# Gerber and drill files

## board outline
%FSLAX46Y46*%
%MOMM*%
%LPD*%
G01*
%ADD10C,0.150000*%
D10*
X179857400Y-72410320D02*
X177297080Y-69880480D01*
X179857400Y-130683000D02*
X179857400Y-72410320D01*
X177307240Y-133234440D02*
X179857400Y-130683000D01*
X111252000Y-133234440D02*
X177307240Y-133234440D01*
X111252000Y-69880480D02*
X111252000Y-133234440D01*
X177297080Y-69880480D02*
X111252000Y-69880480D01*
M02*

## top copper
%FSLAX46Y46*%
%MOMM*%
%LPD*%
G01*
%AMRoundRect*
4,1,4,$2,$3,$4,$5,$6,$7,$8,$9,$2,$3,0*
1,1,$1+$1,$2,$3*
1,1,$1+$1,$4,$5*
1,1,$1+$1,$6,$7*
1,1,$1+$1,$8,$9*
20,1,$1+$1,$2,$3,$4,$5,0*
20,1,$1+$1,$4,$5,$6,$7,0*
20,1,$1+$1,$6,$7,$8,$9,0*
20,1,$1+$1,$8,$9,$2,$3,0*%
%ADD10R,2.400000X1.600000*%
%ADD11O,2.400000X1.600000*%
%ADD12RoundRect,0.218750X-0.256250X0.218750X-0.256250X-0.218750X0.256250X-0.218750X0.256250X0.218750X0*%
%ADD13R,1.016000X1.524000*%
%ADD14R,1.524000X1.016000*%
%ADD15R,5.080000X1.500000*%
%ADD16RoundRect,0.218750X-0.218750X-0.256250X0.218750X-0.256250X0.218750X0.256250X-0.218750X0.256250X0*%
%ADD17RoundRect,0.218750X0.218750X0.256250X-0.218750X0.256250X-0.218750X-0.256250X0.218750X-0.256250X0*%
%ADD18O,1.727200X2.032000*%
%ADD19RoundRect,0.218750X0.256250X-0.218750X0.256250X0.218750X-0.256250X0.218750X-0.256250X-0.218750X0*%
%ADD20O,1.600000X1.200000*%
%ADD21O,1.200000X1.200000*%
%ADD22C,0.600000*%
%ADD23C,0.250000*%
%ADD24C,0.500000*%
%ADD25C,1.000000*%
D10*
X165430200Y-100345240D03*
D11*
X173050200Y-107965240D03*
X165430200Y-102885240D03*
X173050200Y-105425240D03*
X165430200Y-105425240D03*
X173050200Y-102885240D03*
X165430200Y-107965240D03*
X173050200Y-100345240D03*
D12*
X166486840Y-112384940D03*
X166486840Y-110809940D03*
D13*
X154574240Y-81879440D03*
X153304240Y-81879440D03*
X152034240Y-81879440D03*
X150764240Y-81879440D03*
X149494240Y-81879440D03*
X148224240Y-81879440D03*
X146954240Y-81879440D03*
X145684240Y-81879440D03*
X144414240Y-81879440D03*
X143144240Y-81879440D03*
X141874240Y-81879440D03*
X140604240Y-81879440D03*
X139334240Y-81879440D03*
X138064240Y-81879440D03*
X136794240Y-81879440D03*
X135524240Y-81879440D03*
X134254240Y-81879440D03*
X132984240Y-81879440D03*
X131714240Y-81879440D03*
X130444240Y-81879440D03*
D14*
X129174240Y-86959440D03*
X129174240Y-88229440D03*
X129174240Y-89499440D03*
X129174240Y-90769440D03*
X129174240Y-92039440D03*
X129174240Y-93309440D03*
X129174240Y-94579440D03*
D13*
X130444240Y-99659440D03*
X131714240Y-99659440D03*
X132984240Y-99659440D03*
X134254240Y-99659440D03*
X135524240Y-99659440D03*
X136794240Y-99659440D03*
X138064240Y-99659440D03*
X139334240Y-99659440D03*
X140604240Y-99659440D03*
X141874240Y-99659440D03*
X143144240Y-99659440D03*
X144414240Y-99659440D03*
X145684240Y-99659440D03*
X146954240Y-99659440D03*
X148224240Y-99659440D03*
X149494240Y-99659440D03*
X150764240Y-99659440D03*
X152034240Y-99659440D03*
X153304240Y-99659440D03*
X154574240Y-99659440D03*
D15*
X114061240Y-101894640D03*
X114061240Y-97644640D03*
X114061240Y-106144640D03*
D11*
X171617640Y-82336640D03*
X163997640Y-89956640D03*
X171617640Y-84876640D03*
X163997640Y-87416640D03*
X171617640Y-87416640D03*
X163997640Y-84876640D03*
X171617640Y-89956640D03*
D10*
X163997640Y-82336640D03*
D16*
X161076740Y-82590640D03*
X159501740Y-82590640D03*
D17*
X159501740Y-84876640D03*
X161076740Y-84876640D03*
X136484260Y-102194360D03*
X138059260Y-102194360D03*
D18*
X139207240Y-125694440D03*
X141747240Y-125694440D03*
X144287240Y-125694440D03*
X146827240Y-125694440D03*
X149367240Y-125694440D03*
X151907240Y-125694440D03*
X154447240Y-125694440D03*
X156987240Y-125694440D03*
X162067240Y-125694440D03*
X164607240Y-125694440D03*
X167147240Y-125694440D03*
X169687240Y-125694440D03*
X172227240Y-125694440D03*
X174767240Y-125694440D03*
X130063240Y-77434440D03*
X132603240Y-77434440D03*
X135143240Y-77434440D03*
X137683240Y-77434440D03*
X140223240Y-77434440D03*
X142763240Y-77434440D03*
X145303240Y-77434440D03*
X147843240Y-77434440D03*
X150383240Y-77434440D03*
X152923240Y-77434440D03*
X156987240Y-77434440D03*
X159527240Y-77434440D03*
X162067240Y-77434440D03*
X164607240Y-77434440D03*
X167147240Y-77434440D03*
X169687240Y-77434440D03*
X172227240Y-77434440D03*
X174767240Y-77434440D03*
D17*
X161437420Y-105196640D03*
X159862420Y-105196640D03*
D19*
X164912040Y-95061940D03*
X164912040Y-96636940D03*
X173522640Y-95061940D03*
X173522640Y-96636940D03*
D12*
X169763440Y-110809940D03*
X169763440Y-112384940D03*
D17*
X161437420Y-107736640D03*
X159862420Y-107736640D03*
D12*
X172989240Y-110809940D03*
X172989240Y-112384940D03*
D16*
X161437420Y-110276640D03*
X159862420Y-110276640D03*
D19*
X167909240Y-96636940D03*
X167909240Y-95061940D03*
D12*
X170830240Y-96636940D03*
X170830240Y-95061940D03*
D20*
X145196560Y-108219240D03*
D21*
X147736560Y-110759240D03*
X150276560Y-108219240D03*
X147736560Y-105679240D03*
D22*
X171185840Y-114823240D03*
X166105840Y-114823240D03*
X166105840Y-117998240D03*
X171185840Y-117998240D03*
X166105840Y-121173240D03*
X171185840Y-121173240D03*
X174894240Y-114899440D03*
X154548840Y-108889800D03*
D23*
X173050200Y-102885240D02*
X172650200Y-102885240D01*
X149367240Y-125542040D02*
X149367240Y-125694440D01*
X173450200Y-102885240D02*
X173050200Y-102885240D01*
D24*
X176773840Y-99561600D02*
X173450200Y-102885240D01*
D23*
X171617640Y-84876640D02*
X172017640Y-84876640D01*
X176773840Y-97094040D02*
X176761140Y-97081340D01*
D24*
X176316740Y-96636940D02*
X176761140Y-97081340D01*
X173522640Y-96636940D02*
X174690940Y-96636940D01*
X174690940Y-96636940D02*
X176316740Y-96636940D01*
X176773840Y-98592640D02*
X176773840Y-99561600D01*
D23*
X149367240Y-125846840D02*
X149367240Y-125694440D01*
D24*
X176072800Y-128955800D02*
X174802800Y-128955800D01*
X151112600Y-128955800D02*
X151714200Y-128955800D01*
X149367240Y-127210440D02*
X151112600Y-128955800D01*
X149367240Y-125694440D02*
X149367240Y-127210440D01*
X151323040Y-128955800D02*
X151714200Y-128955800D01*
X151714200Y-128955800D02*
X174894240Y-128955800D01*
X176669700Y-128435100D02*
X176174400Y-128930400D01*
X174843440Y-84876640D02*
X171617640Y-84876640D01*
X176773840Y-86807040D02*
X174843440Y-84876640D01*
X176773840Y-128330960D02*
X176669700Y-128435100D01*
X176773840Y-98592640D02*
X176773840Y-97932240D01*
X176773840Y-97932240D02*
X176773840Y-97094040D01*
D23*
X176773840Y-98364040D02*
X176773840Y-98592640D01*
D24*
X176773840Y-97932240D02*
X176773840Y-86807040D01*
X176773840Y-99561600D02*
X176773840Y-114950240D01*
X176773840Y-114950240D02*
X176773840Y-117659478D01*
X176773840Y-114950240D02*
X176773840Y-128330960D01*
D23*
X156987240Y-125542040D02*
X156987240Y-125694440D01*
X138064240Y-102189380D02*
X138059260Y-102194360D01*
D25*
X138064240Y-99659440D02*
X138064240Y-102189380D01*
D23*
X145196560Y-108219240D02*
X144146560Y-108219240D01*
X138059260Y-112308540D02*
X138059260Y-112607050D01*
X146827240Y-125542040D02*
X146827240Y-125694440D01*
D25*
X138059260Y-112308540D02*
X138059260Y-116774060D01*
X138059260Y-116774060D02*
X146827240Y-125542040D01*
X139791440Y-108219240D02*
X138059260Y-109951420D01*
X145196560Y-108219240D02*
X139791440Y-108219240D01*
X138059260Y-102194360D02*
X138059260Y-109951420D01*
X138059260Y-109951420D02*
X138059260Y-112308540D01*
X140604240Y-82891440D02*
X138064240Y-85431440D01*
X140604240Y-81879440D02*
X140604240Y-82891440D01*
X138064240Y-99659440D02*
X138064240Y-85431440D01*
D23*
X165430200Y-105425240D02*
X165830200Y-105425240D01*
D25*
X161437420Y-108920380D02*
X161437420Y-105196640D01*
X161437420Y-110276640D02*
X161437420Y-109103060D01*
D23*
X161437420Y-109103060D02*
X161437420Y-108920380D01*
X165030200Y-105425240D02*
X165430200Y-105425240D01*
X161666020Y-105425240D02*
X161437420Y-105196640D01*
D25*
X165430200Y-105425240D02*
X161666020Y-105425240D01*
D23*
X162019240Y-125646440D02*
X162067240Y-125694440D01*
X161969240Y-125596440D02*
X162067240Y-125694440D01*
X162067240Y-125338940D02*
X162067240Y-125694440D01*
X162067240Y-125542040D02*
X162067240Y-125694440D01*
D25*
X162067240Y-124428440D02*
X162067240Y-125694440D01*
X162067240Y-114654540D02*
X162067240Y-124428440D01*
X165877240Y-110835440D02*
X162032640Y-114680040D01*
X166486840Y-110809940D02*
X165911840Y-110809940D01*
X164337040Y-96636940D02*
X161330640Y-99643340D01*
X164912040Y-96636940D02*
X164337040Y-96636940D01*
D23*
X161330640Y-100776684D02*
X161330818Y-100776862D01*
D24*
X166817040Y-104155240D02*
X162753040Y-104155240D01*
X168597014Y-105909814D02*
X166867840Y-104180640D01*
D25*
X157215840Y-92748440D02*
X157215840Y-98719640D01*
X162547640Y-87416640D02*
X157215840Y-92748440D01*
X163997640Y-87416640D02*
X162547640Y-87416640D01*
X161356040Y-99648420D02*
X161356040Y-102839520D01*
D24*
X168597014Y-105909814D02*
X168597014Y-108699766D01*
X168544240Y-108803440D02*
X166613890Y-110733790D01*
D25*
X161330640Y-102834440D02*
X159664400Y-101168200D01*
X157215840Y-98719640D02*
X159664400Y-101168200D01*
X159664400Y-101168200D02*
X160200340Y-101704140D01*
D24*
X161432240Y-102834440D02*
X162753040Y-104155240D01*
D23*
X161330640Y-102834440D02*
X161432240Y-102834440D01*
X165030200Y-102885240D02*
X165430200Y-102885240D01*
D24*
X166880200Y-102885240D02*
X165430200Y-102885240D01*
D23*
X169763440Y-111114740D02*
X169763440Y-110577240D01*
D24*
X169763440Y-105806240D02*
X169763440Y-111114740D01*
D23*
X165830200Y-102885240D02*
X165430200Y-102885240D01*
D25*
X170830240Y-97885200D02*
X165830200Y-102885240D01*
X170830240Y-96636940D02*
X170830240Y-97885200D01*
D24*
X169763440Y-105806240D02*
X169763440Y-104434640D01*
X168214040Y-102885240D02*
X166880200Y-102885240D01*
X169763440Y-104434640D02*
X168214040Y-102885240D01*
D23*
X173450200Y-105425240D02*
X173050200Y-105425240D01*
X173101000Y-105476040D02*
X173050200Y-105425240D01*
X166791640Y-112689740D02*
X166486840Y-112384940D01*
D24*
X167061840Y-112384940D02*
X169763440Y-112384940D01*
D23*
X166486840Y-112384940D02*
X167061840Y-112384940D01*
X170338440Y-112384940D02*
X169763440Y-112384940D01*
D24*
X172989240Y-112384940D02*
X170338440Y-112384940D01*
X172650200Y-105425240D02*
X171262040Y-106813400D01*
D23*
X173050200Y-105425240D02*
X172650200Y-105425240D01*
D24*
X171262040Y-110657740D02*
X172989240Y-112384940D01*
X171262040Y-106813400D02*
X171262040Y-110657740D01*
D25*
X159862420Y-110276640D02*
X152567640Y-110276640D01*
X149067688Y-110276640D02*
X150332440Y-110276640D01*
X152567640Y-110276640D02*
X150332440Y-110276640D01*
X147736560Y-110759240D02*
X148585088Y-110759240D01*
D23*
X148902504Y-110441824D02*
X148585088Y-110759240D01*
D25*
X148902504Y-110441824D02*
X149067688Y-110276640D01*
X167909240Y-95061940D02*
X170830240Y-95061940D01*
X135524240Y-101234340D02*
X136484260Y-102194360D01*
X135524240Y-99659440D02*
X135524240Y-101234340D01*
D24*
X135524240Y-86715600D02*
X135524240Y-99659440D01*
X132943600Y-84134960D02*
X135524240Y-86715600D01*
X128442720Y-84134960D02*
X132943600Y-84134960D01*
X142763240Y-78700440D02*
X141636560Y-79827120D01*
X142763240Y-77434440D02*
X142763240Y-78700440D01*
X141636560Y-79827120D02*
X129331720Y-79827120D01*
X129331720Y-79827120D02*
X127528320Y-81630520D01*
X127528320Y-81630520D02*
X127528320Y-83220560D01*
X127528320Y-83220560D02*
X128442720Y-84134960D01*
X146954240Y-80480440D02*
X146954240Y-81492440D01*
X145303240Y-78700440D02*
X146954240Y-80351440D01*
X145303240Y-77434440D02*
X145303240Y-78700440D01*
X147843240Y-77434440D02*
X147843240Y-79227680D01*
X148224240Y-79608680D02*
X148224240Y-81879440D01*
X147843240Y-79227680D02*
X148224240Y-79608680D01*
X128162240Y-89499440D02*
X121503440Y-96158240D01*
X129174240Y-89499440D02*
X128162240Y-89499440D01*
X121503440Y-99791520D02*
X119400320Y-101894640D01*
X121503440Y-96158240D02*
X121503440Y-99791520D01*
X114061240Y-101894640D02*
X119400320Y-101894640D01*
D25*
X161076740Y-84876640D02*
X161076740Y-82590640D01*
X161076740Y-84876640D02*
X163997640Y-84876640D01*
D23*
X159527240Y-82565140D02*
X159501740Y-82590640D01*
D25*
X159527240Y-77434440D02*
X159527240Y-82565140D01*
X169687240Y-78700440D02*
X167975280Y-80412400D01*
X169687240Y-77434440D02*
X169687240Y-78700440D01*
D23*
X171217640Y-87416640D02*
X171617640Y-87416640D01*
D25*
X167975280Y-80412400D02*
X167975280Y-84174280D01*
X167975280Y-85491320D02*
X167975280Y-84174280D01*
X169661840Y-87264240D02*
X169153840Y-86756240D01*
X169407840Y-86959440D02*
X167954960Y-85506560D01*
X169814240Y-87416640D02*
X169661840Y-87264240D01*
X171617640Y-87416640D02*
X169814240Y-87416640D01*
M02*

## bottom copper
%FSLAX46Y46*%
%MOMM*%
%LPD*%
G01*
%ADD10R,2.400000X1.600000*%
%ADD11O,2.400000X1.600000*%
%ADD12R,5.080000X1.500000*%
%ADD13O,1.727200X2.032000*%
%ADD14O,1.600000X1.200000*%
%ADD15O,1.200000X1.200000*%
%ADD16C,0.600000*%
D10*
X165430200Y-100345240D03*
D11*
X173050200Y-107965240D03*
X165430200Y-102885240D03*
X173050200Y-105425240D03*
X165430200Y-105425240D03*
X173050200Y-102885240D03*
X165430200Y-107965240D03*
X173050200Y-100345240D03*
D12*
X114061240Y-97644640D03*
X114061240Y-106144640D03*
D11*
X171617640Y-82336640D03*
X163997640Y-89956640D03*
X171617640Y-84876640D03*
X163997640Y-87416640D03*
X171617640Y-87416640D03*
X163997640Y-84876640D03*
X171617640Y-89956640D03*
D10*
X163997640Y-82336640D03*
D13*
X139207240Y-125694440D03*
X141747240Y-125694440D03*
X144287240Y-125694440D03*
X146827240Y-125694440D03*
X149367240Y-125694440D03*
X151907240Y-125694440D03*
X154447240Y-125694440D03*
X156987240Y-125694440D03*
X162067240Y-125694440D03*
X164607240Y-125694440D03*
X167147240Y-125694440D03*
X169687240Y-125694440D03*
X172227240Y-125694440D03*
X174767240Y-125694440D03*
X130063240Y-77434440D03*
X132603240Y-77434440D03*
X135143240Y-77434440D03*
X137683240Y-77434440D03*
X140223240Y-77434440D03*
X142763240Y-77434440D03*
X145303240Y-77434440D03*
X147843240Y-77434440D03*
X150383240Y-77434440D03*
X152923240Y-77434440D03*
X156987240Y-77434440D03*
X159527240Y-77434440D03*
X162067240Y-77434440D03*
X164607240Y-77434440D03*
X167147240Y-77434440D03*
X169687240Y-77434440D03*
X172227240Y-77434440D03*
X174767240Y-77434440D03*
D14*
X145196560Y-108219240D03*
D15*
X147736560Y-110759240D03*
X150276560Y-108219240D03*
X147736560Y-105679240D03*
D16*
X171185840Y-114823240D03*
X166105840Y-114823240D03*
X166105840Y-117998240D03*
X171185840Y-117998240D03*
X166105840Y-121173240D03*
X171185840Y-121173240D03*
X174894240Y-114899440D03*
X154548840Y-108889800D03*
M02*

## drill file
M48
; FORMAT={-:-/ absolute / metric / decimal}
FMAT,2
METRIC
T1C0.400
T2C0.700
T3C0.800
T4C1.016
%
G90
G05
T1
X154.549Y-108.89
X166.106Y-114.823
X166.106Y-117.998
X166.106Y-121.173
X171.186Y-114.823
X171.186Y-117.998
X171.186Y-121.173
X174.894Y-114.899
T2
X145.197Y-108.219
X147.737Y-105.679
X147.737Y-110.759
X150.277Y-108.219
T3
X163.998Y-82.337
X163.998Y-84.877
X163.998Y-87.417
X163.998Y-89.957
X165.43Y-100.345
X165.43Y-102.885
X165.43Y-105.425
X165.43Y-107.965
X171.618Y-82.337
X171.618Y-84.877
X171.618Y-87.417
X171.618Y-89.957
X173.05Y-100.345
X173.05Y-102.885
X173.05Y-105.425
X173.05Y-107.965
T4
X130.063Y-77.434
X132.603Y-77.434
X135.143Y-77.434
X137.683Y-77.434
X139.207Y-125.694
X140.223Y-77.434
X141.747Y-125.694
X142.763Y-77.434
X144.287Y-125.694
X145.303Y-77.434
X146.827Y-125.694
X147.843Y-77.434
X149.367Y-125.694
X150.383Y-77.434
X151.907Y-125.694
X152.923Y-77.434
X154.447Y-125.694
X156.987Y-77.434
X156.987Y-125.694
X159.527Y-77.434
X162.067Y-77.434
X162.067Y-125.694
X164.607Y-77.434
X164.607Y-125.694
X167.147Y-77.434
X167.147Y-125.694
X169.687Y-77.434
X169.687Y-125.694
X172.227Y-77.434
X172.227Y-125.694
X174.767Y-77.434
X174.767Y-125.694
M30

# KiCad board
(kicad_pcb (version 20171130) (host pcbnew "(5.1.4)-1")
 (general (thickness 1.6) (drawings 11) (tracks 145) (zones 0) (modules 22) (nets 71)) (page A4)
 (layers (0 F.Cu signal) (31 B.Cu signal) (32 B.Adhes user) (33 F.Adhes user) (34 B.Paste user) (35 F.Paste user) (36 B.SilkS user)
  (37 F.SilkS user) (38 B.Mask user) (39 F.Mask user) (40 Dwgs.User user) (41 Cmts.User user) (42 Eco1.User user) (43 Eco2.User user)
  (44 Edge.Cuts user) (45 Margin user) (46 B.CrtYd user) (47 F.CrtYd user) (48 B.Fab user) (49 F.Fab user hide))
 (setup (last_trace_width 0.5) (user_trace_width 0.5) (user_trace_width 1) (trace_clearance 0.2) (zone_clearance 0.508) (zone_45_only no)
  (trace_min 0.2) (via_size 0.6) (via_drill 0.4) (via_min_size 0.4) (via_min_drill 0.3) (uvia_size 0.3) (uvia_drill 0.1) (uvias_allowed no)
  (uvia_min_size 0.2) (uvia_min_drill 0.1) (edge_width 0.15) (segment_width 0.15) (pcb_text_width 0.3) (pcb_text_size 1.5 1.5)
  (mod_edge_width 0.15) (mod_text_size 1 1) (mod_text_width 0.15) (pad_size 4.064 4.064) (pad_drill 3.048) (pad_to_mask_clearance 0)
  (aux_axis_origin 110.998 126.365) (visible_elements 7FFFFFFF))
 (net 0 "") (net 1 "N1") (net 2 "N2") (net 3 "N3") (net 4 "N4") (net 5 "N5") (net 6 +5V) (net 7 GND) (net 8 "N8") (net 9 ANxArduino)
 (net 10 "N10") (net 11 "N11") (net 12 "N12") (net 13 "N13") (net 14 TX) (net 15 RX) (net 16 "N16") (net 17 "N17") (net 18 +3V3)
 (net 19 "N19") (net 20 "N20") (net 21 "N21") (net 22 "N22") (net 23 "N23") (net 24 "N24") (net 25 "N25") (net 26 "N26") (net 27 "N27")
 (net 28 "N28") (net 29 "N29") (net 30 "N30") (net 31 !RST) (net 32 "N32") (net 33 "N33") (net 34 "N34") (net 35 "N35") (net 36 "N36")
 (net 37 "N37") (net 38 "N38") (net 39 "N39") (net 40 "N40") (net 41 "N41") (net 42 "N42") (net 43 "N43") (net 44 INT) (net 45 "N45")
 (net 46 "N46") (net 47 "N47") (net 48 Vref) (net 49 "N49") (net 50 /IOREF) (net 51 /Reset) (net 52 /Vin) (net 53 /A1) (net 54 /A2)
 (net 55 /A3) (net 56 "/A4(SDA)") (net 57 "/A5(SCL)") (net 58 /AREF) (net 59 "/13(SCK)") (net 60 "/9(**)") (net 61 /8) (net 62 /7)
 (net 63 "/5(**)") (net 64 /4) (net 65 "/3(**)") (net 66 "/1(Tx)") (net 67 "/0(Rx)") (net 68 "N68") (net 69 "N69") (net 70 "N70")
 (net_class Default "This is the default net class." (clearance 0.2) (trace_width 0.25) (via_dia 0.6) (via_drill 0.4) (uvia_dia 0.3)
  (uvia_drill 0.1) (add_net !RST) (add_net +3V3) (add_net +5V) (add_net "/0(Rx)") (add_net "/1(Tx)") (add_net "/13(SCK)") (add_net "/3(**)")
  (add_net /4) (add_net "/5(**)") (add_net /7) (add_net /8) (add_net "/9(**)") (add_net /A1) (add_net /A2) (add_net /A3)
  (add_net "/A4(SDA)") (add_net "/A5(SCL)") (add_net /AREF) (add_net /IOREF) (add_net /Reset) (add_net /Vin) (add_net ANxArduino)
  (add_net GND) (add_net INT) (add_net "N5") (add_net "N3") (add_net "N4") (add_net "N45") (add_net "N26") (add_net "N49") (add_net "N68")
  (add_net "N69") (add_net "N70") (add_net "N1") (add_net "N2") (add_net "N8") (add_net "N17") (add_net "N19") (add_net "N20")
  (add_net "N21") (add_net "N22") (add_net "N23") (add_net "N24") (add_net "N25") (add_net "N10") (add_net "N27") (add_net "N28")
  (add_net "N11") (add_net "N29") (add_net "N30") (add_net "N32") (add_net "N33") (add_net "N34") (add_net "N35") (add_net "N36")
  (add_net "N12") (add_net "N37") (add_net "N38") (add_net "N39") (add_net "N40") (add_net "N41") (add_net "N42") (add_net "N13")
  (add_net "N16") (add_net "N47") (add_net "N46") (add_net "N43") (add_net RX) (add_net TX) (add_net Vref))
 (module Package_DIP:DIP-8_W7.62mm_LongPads (layer F.Cu) (at 165.4302 100.34524)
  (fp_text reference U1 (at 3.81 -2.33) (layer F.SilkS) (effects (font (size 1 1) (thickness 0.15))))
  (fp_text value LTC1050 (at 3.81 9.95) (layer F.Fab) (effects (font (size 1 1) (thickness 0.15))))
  (pad 1 thru_hole rect (at 0 0) (size 2.4 1.6) (drill 0.8) (layers *.Cu *.Mask) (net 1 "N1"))
  (pad 5 thru_hole oval (at 7.62 7.62) (size 2.4 1.6) (drill 0.8) (layers *.Cu *.Mask) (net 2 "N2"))
  (pad 2 thru_hole oval (at 0 2.54) (size 2.4 1.6) (drill 0.8) (layers *.Cu *.Mask) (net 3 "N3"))
  (pad 6 thru_hole oval (at 7.62 5.08) (size 2.4 1.6) (drill 0.8) (layers *.Cu *.Mask) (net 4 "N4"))
  (pad 3 thru_hole oval (at 0 5.08) (size 2.4 1.6) (drill 0.8) (layers *.Cu *.Mask) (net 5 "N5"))
  (pad 7 thru_hole oval (at 7.62 2.54) (size 2.4 1.6) (drill 0.8) (layers *.Cu *.Mask) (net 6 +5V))
  (pad 4 thru_hole oval (at 0 7.62) (size 2.4 1.6) (drill 0.8) (layers *.Cu *.Mask) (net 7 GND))
  (pad 8 thru_hole oval (at 7.62 0) (size 2.4 1.6) (drill 0.8) (layers *.Cu *.Mask) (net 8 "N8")))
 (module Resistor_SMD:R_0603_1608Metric (layer F.Cu) (at 166.48684 111.59744 270)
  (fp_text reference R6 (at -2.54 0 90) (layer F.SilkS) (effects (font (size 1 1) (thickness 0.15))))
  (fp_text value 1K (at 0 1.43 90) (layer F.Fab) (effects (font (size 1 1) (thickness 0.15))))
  (pad 2 smd roundrect (at 0.7875 0 270) (size 0.875 0.95) (layers F.Cu F.Paste F.Mask) (roundrect_rratio 0.25) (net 4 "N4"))
  (pad 1 smd roundrect (at -0.7875 0 270) (size 0.875 0.95) (layers F.Cu F.Paste F.Mask) (roundrect_rratio 0.25) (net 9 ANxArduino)))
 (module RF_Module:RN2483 (layer F.Cu) (at 142.50924 90.76944 270)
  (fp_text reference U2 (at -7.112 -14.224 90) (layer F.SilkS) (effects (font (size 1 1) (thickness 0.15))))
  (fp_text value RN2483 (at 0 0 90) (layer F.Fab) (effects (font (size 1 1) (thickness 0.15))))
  (pad 1 smd rect (at -8.89 -12.065 270) (size 1.524 1.016) (layers F.Cu F.Paste F.Mask) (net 7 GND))
  (pad 2 smd rect (at -8.89 -10.795 270) (size 1.524 1.016) (layers F.Cu F.Paste F.Mask) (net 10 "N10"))
  (pad 3 smd rect (at -8.89 -9.525 270) (size 1.524 1.016) (layers F.Cu F.Paste F.Mask) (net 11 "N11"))
  (pad 4 smd rect (at -8.89 -8.255 270) (size 1.524 1.016) (layers F.Cu F.Paste F.Mask) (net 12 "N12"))
  (pad 5 smd rect (at -8.89 -6.985 270) (size 1.524 1.016) (layers F.Cu F.Paste F.Mask) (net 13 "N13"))
  (pad 6 smd rect (at -8.89 -5.715 270) (size 1.524 1.016) (layers F.Cu F.Paste F.Mask) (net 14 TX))
  (pad 7 smd rect (at -8.89 -4.445 270) (size 1.524 1.016) (layers F.Cu F.Paste F.Mask) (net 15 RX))
  (pad 8 smd rect (at -8.89 -3.175 270) (size 1.524 1.016) (layers F.Cu F.Paste F.Mask) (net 7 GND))
  (pad 9 smd rect (at -8.89 -1.905 270) (size 1.524 1.016) (layers F.Cu F.Paste F.Mask) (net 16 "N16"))
  (pad 10 smd rect (at -8.89 -0.635 270) (size 1.524 1.016) (layers F.Cu F.Paste F.Mask) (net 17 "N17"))
  (pad 11 smd rect (at -8.89 0.635 270) (size 1.524 1.016) (layers F.Cu F.Paste F.Mask) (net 7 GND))
  (pad 12 smd rect (at -8.89 1.905 270) (size 1.524 1.016) (layers F.Cu F.Paste F.Mask) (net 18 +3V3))
  (pad 13 smd rect (at -8.89 3.175 270) (size 1.524 1.016) (layers F.Cu F.Paste F.Mask) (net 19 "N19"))
  (pad 14 smd rect (at -8.89 4.445 270) (size 1.524 1.016) (layers F.Cu F.Paste F.Mask) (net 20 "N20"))
  (pad 15 smd rect (at -8.89 5.715 270) (size 1.524 1.016) (layers F.Cu F.Paste F.Mask) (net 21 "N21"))
  (pad 16 smd rect (at -8.89 6.985 270) (size 1.524 1.016) (layers F.Cu F.Paste F.Mask) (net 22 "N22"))
  (pad 17 smd rect (at -8.89 8.255 270) (size 1.524 1.016) (layers F.Cu F.Paste F.Mask) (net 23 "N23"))
  (pad 18 smd rect (at -8.89 9.525 270) (size 1.524 1.016) (layers F.Cu F.Paste F.Mask) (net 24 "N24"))
  (pad 19 smd rect (at -8.89 10.795 270) (size 1.524 1.016) (layers F.Cu F.Paste F.Mask) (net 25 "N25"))
  (pad 20 smd rect (at -8.89 12.065 270) (size 1.524 1.016) (layers F.Cu F.Paste F.Mask) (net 7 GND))
  (pad 21 smd rect (at -3.81 13.335) (size 1.524 1.016) (layers F.Cu F.Paste F.Mask) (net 7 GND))
  (pad 22 smd rect (at -2.54 13.335) (size 1.524 1.016) (layers F.Cu F.Paste F.Mask) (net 7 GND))
  (pad 23 smd rect (at -1.27 13.335) (size 1.524 1.016) (layers F.Cu F.Paste F.Mask) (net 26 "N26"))
  (pad 24 smd rect (at 0 13.335) (size 1.524 1.016) (layers F.Cu F.Paste F.Mask) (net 7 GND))
  (pad 25 smd rect (at 1.27 13.335) (size 1.524 1.016) (layers F.Cu F.Paste F.Mask) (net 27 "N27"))
  (pad 26 smd rect (at 2.54 13.335) (size 1.524 1.016) (layers F.Cu F.Paste F.Mask) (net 7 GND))
  (pad 27 smd rect (at 3.81 13.335) (size 1.524 1.016) (layers F.Cu F.Paste F.Mask) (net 7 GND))
  (pad 28 smd rect (at 8.89 12.065 270) (size 1.524 1.016) (layers F.Cu F.Paste F.Mask) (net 7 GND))
  (pad 29 smd rect (at 8.89 10.795 270) (size 1.524 1.016) (layers F.Cu F.Paste F.Mask) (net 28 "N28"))
  (pad 30 smd rect (at 8.89 9.525 270) (size 1.524 1.016) (layers F.Cu F.Paste F.Mask) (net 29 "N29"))
  (pad 31 smd rect (at 8.89 8.255 270) (size 1.524 1.016) (layers F.Cu F.Paste F.Mask) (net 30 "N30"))
  (pad 32 smd rect (at 8.89 6.985 270) (size 1.524 1.016) (layers F.Cu F.Paste F.Mask) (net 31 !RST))
  (pad 33 smd rect (at 8.89 5.715 270) (size 1.524 1.016) (layers F.Cu F.Paste F.Mask) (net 7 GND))
  (pad 34 smd rect (at 8.89 4.445 270) (size 1.524 1.016) (layers F.Cu F.Paste F.Mask) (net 18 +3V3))
  (pad 35 smd rect (at 8.89 3.175 270) (size 1.524 1.016) (layers F.Cu F.Paste F.Mask) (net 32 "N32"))
  (pad 36 smd rect (at 8.89 1.905 270) (size 1.524 1.016) (layers F.Cu F.Paste F.Mask) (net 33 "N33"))
  (pad 37 smd rect (at 8.89 0.635 270) (size 1.524 1.016) (layers F.Cu F.Paste F.Mask) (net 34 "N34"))
  (pad 38 smd rect (at 8.89 -0.635 270) (size 1.524 1.016) (layers F.Cu F.Paste F.Mask) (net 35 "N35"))
  (pad 39 smd rect (at 8.89 -1.905 270) (size 1.524 1.016) (layers F.Cu F.Paste F.Mask) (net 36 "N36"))
  (pad 40 smd rect (at 8.89 -3.175 270) (size 1.524 1.016) (layers F.Cu F.Paste F.Mask) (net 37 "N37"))
  (pad 41 smd rect (at 8.89 -4.445 270) (size 1.524 1.016) (layers F.Cu F.Paste F.Mask) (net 7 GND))
  (pad 42 smd rect (at 8.89 -5.715 270) (size 1.524 1.016) (layers F.Cu F.Paste F.Mask) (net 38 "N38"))
  (pad 43 smd rect (at 8.89 -6.985 270) (size 1.524 1.016) (layers F.Cu F.Paste F.Mask) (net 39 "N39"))
  (pad 44 smd rect (at 8.89 -8.255 270) (size 1.524 1.016) (layers F.Cu F.Paste F.Mask) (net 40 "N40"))
  (pad 45 smd rect (at 8.89 -9.525 270) (size 1.524 1.016) (layers F.Cu F.Paste F.Mask) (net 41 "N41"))
  (pad 46 smd rect (at 8.89 -10.795 270) (size 1.524 1.016) (layers F.Cu F.Paste F.Mask) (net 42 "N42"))
  (pad 47 smd rect (at 8.89 -12.065 270) (size 1.524 1.016) (layers F.Cu F.Paste F.Mask) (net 7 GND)))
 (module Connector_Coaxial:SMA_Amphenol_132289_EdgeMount (layer F.Cu) (at 114.06124 101.89464)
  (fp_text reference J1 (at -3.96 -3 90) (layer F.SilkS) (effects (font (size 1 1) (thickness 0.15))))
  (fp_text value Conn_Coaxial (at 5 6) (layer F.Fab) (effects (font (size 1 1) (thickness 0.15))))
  (pad 1 smd rect (at 0 0 90) (size 1.5 5.08) (layers F.Cu F.Paste F.Mask) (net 26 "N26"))
  (pad 2 smd rect (at 0 -4.25 90) (size 1.5 5.08) (layers F.Cu F.Paste F.Mask) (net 7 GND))
  (pad 2 smd rect (at 0 4.25 90) (size 1.5 5.08) (layers F.Cu F.Paste F.Mask) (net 7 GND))
  (pad 2 smd rect (at 0 -4.25 90) (size 1.5 5.08) (layers B.Cu B.Paste B.Mask) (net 7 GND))
  (pad 2 smd rect (at 0 4.25 90) (size 1.5 5.08) (layers B.Cu B.Paste B.Mask) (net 7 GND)))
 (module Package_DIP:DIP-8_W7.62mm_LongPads (layer F.Cu) (at 163.99764 82.33664)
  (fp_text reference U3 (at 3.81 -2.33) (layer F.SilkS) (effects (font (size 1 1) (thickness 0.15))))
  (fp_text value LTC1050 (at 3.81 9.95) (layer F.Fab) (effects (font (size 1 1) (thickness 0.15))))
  (pad 8 thru_hole oval (at 7.62 0) (size 2.4 1.6) (drill 0.8) (layers *.Cu *.Mask) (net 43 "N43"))
  (pad 4 thru_hole oval (at 0 7.62) (size 2.4 1.6) (drill 0.8) (layers *.Cu *.Mask) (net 7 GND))
  (pad 7 thru_hole oval (at 7.62 2.54) (size 2.4 1.6) (drill 0.8) (layers *.Cu *.Mask) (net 6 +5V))
  (pad 3 thru_hole oval (at 0 5.08) (size 2.4 1.6) (drill 0.8) (layers *.Cu *.Mask) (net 9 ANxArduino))
  (pad 6 thru_hole oval (at 7.62 5.08) (size 2.4 1.6) (drill 0.8) (layers *.Cu *.Mask) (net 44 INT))
  (pad 2 thru_hole oval (at 0 2.54) (size 2.4 1.6) (drill 0.8) (layers *.Cu *.Mask) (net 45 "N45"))
  (pad 5 thru_hole oval (at 7.62 7.62) (size 2.4 1.6) (drill 0.8) (layers *.Cu *.Mask) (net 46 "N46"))
  (pad 1 thru_hole rect (at 0 0) (size 2.4 1.6) (drill 0.8) (layers *.Cu *.Mask) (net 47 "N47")))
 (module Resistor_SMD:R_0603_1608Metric (layer F.Cu) (at 160.28924 82.59064)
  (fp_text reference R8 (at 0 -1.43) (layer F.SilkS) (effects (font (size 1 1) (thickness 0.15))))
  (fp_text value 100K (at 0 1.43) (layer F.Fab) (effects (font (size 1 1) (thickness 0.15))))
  (pad 2 smd roundrect (at 0.7875 0) (size 0.875 0.95) (layers F.Cu F.Paste F.Mask) (roundrect_rratio 0.25) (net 45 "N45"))
  (pad 1 smd roundrect (at -0.7875 0) (size 0.875 0.95) (layers F.Cu F.Paste F.Mask) (roundrect_rratio 0.25) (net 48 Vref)))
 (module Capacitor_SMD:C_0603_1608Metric (layer F.Cu) (at 160.28924 84.87664 180)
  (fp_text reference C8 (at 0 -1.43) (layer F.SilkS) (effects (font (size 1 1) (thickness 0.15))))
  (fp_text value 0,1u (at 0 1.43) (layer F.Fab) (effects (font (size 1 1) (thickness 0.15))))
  (pad 2 smd roundrect (at 0.7875 0 180) (size 0.875 0.95) (layers F.Cu F.Paste F.Mask) (roundrect_rratio 0.25) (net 7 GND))
  (pad 1 smd roundrect (at -0.7875 0 180) (size 0.875 0.95) (layers F.Cu F.Paste F.Mask) (roundrect_rratio 0.25) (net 45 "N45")))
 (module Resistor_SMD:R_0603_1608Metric (layer F.Cu) (at 137.27176 102.19436 180)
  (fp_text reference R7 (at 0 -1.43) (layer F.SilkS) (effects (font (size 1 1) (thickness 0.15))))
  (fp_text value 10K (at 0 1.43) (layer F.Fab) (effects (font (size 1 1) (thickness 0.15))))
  (pad 2 smd roundrect (at 0.7875 0 180) (size 0.875 0.95) (layers F.Cu F.Paste F.Mask) (roundrect_rratio 0.25) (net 31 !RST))
  (pad 1 smd roundrect (at -0.7875 0 180) (size 0.875 0.95) (layers F.Cu F.Paste F.Mask) (roundrect_rratio 0.25) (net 18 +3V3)))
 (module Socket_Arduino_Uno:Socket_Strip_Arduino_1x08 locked (layer F.Cu) (at 139.20724 125.69444)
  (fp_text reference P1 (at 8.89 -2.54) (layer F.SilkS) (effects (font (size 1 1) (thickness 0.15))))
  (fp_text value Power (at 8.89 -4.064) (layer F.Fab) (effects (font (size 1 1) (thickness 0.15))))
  (pad 1 thru_hole oval (at 0 0) (size 1.7272 2.032) (drill 1.016) (layers *.Cu *.Mask F.SilkS) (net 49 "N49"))
  (pad 2 thru_hole oval (at 2.54 0) (size 1.7272 2.032) (drill 1.016) (layers *.Cu *.Mask F.SilkS) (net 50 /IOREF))
  (pad 3 thru_hole oval (at 5.08 0) (size 1.7272 2.032) (drill 1.016) (layers *.Cu *.Mask F.SilkS) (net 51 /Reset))
  (pad 4 thru_hole oval (at 7.62 0) (size 1.7272 2.032) (drill 1.016) (layers *.Cu *.Mask F.SilkS) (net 18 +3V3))
  (pad 5 thru_hole oval (at 10.16 0) (size 1.7272 2.032) (drill 1.016) (layers *.Cu *.Mask F.SilkS) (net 6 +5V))
  (pad 6 thru_hole oval (at 12.7 0) (size 1.7272 2.032) (drill 1.016) (layers *.Cu *.Mask F.SilkS) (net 7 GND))
  (pad 7 thru_hole oval (at 15.24 0) (size 1.7272 2.032) (drill 1.016) (layers *.Cu *.Mask F.SilkS) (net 7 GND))
  (pad 8 thru_hole oval (at 17.78 0) (size 1.7272 2.032) (drill 1.016) (layers *.Cu *.Mask F.SilkS) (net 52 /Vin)))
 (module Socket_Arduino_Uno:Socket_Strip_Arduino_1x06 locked (layer F.Cu) (at 162.06724 125.69444)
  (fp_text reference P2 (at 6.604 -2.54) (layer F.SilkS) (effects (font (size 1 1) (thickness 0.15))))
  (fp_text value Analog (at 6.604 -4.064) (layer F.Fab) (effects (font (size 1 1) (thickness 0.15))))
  (pad 1 thru_hole oval (at 0 0) (size 1.7272 2.032) (drill 1.016) (layers *.Cu *.Mask F.SilkS) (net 9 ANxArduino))
  (pad 2 thru_hole oval (at 2.54 0) (size 1.7272 2.032) (drill 1.016) (layers *.Cu *.Mask F.SilkS) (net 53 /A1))
  (pad 3 thru_hole oval (at 5.08 0) (size 1.7272 2.032) (drill 1.016) (layers *.Cu *.Mask F.SilkS) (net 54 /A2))
  (pad 4 thru_hole oval (at 7.62 0) (size 1.7272 2.032) (drill 1.016) (layers *.Cu *.Mask F.SilkS) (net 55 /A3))
  (pad 5 thru_hole oval (at 10.16 0) (size 1.7272 2.032) (drill 1.016) (layers *.Cu *.Mask F.SilkS) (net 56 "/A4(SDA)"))
  (pad 6 thru_hole oval (at 12.7 0) (size 1.7272 2.032) (drill 1.016) (layers *.Cu *.Mask F.SilkS) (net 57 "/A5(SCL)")))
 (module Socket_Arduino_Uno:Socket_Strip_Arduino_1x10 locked (layer F.Cu) (at 130.06324 77.43444)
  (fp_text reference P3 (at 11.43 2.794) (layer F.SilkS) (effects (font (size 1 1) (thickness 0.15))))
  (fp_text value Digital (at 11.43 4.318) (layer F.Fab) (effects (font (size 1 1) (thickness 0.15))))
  (pad 1 thru_hole oval (at 0 0) (size 1.7272 2.032) (drill 1.016) (layers *.Cu *.Mask F.SilkS) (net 57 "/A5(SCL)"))
  (pad 2 thru_hole oval (at 2.54 0) (size 1.7272 2.032) (drill 1.016) (layers *.Cu *.Mask F.SilkS) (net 56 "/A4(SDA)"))
  (pad 3 thru_hole oval (at 5.08 0) (size 1.7272 2.032) (drill 1.016) (layers *.Cu *.Mask F.SilkS) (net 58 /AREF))
  (pad 4 thru_hole oval (at 7.62 0) (size 1.7272 2.032) (drill 1.016) (layers *.Cu *.Mask F.SilkS) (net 7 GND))
  (pad 5 thru_hole oval (at 10.16 0) (size 1.7272 2.032) (drill 1.016) (layers *.Cu *.Mask F.SilkS) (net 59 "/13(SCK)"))
  (pad 6 thru_hole oval (at 12.7 0) (size 1.7272 2.032) (drill 1.016) (layers *.Cu *.Mask F.SilkS) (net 31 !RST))
  (pad 7 thru_hole oval (at 15.24 0) (size 1.7272 2.032) (drill 1.016) (layers *.Cu *.Mask F.SilkS) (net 15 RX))
  (pad 8 thru_hole oval (at 17.78 0) (size 1.7272 2.032) (drill 1.016) (layers *.Cu *.Mask F.SilkS) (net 14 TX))
  (pad 9 thru_hole oval (at 20.32 0) (size 1.7272 2.032) (drill 1.016) (layers *.Cu *.Mask F.SilkS) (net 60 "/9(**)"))
  (pad 10 thru_hole oval (at 22.86 0) (size 1.7272 2.032) (drill 1.016) (layers *.Cu *.Mask F.SilkS) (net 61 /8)))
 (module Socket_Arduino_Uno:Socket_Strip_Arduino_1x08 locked (layer F.Cu) (at 156.98724 77.43444)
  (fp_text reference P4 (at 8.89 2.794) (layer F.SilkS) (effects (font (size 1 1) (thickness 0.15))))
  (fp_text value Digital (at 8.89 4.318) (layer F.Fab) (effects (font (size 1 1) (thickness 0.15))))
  (pad 1 thru_hole oval (at 0 0) (size 1.7272 2.032) (drill 1.016) (layers *.Cu *.Mask F.SilkS) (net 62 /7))
  (pad 2 thru_hole oval (at 2.54 0) (size 1.7272 2.032) (drill 1.016) (layers *.Cu *.Mask F.SilkS) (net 48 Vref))
  (pad 3 thru_hole oval (at 5.08 0) (size 1.7272 2.032) (drill 1.016) (layers *.Cu *.Mask F.SilkS) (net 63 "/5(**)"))
  (pad 4 thru_hole oval (at 7.62 0) (size 1.7272 2.032) (drill 1.016) (layers *.Cu *.Mask F.SilkS) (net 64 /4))
  (pad 5 thru_hole oval (at 10.16 0) (size 1.7272 2.032) (drill 1.016) (layers *.Cu *.Mask F.SilkS) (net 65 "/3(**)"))
  (pad 6 thru_hole oval (at 12.7 0) (size 1.7272 2.032) (drill 1.016) (layers *.Cu *.Mask F.SilkS) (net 44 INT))
  (pad 7 thru_hole oval (at 15.24 0) (size 1.7272 2.032) (drill 1.016) (layers *.Cu *.Mask F.SilkS) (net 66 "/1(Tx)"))
  (pad 8 thru_hole oval (at 17.78 0) (size 1.7272 2.032) (drill 1.016) (layers *.Cu *.Mask F.SilkS) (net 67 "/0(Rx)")))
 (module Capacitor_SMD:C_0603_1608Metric (layer F.Cu) (at 160.64992 105.19664 180)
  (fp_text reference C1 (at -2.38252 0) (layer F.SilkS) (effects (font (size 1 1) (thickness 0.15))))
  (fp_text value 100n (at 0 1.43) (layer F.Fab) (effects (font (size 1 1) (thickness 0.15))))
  (pad 1 smd roundrect (at -0.7875 0 180) (size 0.875 0.95) (layers F.Cu F.Paste F.Mask) (roundrect_rratio 0.25) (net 5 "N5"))
  (pad 2 smd roundrect (at 0.7875 0 180) (size 0.875 0.95) (layers F.Cu F.Paste F.Mask) (roundrect_rratio 0.25) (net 7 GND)))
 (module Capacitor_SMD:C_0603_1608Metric (layer F.Cu) (at 164.91204 95.84944 90)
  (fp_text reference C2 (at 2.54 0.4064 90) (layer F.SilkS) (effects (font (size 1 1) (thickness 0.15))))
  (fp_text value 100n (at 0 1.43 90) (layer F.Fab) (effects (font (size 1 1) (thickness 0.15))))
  (pad 2 smd roundrect (at 0.7875 0 90) (size 0.875 0.95) (layers F.Cu F.Paste F.Mask) (roundrect_rratio 0.25) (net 7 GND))
  (pad 1 smd roundrect (at -0.7875 0 90) (size 0.875 0.95) (layers F.Cu F.Paste F.Mask) (roundrect_rratio 0.25) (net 9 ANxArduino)))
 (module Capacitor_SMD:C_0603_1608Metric (layer F.Cu) (at 173.52264 95.84944 90)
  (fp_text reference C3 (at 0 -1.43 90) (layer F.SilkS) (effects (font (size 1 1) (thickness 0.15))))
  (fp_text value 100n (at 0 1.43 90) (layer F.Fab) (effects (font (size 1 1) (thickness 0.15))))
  (pad 2 smd roundrect (at 0.7875 0 90) (size 0.875 0.95) (layers F.Cu F.Paste F.Mask) (roundrect_rratio 0.25) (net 7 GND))
  (pad 1 smd roundrect (at -0.7875 0 90) (size 0.875 0.95) (layers F.Cu F.Paste F.Mask) (roundrect_rratio 0.25) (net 6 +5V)))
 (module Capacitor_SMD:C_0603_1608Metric (layer F.Cu) (at 169.76344 111.59744 270)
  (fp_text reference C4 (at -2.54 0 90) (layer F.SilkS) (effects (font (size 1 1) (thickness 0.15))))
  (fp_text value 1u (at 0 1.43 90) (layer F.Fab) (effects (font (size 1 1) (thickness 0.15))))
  (pad 1 smd roundrect (at -0.7875 0 270) (size 0.875 0.95) (layers F.Cu F.Paste F.Mask) (roundrect_rratio 0.25) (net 3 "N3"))
  (pad 2 smd roundrect (at 0.7875 0 270) (size 0.875 0.95) (layers F.Cu F.Paste F.Mask) (roundrect_rratio 0.25) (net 4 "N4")))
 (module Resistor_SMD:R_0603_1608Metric (layer F.Cu) (at 160.64992 107.73664 180)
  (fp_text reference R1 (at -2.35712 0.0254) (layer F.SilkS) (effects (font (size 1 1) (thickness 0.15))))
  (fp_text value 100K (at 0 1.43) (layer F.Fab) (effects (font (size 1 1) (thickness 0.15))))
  (pad 1 smd roundrect (at -0.7875 0 180) (size 0.875 0.95) (layers F.Cu F.Paste F.Mask) (roundrect_rratio 0.25) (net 5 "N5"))
  (pad 2 smd roundrect (at 0.7875 0 180) (size 0.875 0.95) (layers F.Cu F.Paste F.Mask) (roundrect_rratio 0.25) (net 7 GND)))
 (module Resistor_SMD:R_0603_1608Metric (layer F.Cu) (at 172.98924 111.59744 270)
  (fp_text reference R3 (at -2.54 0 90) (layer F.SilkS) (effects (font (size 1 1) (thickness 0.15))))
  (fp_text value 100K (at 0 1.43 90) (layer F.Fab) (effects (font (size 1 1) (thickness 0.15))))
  (pad 1 smd roundrect (at -0.7875 0 270) (size 0.875 0.95) (layers F.Cu F.Paste F.Mask) (roundrect_rratio 0.25) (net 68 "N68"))
  (pad 2 smd roundrect (at 0.7875 0 270) (size 0.875 0.95) (layers F.Cu F.Paste F.Mask) (roundrect_rratio 0.25) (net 4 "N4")))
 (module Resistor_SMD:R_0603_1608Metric (layer F.Cu) (at 160.64992 110.27664)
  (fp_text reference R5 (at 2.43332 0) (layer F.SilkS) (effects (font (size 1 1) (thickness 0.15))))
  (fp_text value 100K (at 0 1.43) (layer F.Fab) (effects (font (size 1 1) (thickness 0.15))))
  (pad 2 smd roundrect (at 0.7875 0) (size 0.875 0.95) (layers F.Cu F.Paste F.Mask) (roundrect_rratio 0.25) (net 5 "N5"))
  (pad 1 smd roundrect (at -0.7875 0) (size 0.875 0.95) (layers F.Cu F.Paste F.Mask) (roundrect_rratio 0.25) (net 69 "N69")))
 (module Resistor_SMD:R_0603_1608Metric (layer F.Cu) (at 167.90924 95.84944 90)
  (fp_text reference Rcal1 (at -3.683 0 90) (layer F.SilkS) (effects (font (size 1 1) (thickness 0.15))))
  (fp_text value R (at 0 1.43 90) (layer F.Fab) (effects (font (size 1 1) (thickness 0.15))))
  (pad 1 smd roundrect (at -0.7875 0 90) (size 0.875 0.95) (layers F.Cu F.Paste F.Mask) (roundrect_rratio 0.25) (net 7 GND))
  (pad 2 smd roundrect (at 0.7875 0 90) (size 0.875 0.95) (layers F.Cu F.Paste F.Mask) (roundrect_rratio 0.25) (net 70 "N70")))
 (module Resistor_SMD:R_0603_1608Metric (layer F.Cu) (at 170.83024 95.84944 270)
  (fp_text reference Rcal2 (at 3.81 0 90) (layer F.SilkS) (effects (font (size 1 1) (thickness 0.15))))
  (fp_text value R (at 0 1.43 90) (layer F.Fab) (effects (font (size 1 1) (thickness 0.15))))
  (pad 2 smd roundrect (at 0.7875 0 270) (size 0.875 0.95) (layers F.Cu F.Paste F.Mask) (roundrect_rratio 0.25) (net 3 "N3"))
  (pad 1 smd roundrect (at -0.7875 0 270) (size 0.875 0.95) (layers F.Cu F.Paste F.Mask) (roundrect_rratio 0.25) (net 70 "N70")))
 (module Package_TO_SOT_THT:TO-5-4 (layer F.Cu) (at 145.19656 108.21924)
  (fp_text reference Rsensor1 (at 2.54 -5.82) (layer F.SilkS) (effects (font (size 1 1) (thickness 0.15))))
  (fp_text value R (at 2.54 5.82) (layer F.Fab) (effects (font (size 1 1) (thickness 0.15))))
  (pad 1 thru_hole oval (at 0 0) (size 1.6 1.2) (drill 0.7) (layers *.Cu *.Mask) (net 18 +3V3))
  (pad 2 thru_hole oval (at 2.54 2.54) (size 1.2 1.2) (drill 0.7) (layers *.Cu *.Mask) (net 69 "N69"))
  (pad 3 thru_hole oval (at 5.08 0) (size 1.2 1.2) (drill 0.7) (layers *.Cu *.Mask))
  (pad 4 thru_hole oval (at 2.54 -2.54) (size 1.2 1.2) (drill 0.7) (layers *.Cu *.Mask)))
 (gr_line (start 179.8574 72.41032) (end 177.29708 69.88048) (angle 90) (layer Edge.Cuts) (width 0.15))
 (gr_line (start 179.8574 130.683) (end 179.8574 72.41032) (angle 90) (layer Edge.Cuts) (width 0.15))
 (gr_line (start 177.30724 133.23444) (end 179.8574 130.683) (angle 90) (layer Edge.Cuts) (width 0.15))
 (gr_line (start 111.252 133.23444) (end 177.30724 133.23444) (angle 90) (layer Edge.Cuts) (width 0.15))
 (gr_line (start 111.252 69.88048) (end 111.252 133.23444) (angle 90) (layer Edge.Cuts) (width 0.15))
 (gr_line (start 177.29708 69.88048) (end 111.252 69.88048) (angle 90) (layer Edge.Cuts) (width 0.15))
 (segment (start 173.0502 102.88524) (end 172.6502 102.88524) (width 0.25) (layer F.Cu) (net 6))
 (segment (start 149.36724 125.54204) (end 149.36724 125.69444) (width 0.25) (layer F.Cu) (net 6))
 (segment (start 173.4502 102.88524) (end 173.0502 102.88524) (width 0.25) (layer F.Cu) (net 6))
 (segment (start 176.77384 99.5616) (end 173.4502 102.88524) (width 0.5) (layer F.Cu) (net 6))
 (segment (start 171.61764 84.87664) (end 172.01764 84.87664) (width 0.25) (layer F.Cu) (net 6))
 (segment (start 176.77384 97.09404) (end 176.76114 97.08134) (width 0.25) (layer F.Cu) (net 6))
 (segment (start 176.31674 96.63694) (end 176.76114 97.08134) (width 0.5) (layer F.Cu) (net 6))
 (segment (start 173.52264 96.63694) (end 174.69094 96.63694) (width 0.5) (layer F.Cu) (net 6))
 (segment (start 174.69094 96.63694) (end 176.31674 96.63694) (width 0.5) (layer F.Cu) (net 6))
 (segment (start 176.77384 98.59264) (end 176.77384 99.5616) (width 0.5) (layer F.Cu) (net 6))
 (segment (start 149.36724 125.84684) (end 149.36724 125.69444) (width 0.25) (layer F.Cu) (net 6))
 (segment (start 176.0728 128.9558) (end 174.8028 128.9558) (width 0.5) (layer F.Cu) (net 6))
 (segment (start 151.1126 128.9558) (end 151.7142 128.9558) (width 0.5) (layer F.Cu) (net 6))
 (segment (start 149.36724 127.21044) (end 151.1126 128.9558) (width 0.5) (layer F.Cu) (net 6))
 (segment (start 149.36724 125.69444) (end 149.36724 127.21044) (width 0.5) (layer F.Cu) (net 6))
 (segment (start 151.32304 128.9558) (end 151.7142 128.9558) (width 0.5) (layer F.Cu) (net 6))
 (segment (start 151.7142 128.9558) (end 174.89424 128.9558) (width 0.5) (layer F.Cu) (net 6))
 (segment (start 176.6697 128.4351) (end 176.1744 128.9304) (width 0.5) (layer F.Cu) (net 6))
 (segment (start 174.84344 84.87664) (end 171.61764 84.87664) (width 0.5) (layer F.Cu) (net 6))
 (segment (start 176.77384 86.80704) (end 174.84344 84.87664) (width 0.5) (layer F.Cu) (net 6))
 (segment (start 176.77384 128.33096) (end 176.6697 128.4351) (width 0.5) (layer F.Cu) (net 6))
 (segment (start 176.77384 98.59264) (end 176.77384 97.93224) (width 0.5) (layer F.Cu) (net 6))
 (segment (start 176.77384 97.93224) (end 176.77384 97.09404) (width 0.5) (layer F.Cu) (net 6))
 (segment (start 176.77384 98.36404) (end 176.77384 98.59264) (width 0.25) (layer F.Cu) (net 6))
 (segment (start 176.77384 97.93224) (end 176.77384 86.80704) (width 0.5) (layer F.Cu) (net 6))
 (segment (start 176.77384 99.5616) (end 176.77384 114.95024) (width 0.5) (layer F.Cu) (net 6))
 (segment (start 176.77384 114.95024) (end 176.77384 117.659478) (width 0.5) (layer F.Cu) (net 6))
 (segment (start 176.77384 114.95024) (end 176.77384 128.33096) (width 0.5) (layer F.Cu) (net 6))
 (via (at 171.18584 114.82324) (size 0.6) (drill 0.4) (layers F.Cu B.Cu) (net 7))
 (via (at 166.10584 114.82324) (size 0.6) (drill 0.4) (layers F.Cu B.Cu) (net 7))
 (via (at 166.10584 117.99824) (size 0.6) (drill 0.4) (layers F.Cu B.Cu) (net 7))
 (via (at 171.18584 117.99824) (size 0.6) (drill 0.4) (layers F.Cu B.Cu) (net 7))
 (via (at 166.10584 121.17324) (size 0.6) (drill 0.4) (layers F.Cu B.Cu) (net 7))
 (via (at 171.18584 121.17324) (size 0.6) (drill 0.4) (layers F.Cu B.Cu) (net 7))
 (via (at 174.89424 114.89944) (size 0.6) (drill 0.4) (layers F.Cu B.Cu) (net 7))
 (via (at 154.54884 108.8898) (size 0.6) (drill 0.4) (layers F.Cu B.Cu) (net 7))
 (segment (start 156.98724 125.54204) (end 156.98724 125.69444) (width 0.25) (layer F.Cu) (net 52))
 (segment (start 138.06424 102.18938) (end 138.05926 102.19436) (width 0.25) (layer F.Cu) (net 18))
 (segment (start 138.06424 99.65944) (end 138.06424 102.18938) (width 1) (layer F.Cu) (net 18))
 (segment (start 145.19656 108.21924) (end 144.14656 108.21924) (width 0.25) (layer F.Cu) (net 18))
 (segment (start 138.05926 112.30854) (end 138.05926 112.60705) (width 0.25) (layer F.Cu) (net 18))
 (segment (start 146.82724 125.54204) (end 146.82724 125.69444) (width 0.25) (layer F.Cu) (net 18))
 (segment (start 138.05926 112.30854) (end 138.05926 116.77406) (width 1) (layer F.Cu) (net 18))
 (segment (start 138.05926 116.77406) (end 146.82724 125.54204) (width 1) (layer F.Cu) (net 18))
 (segment (start 139.79144 108.21924) (end 138.05926 109.95142) (width 1) (layer F.Cu) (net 18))
 (segment (start 145.19656 108.21924) (end 139.79144 108.21924) (width 1) (layer F.Cu) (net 18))
 (segment (start 138.05926 102.19436) (end 138.05926 109.95142) (width 1) (layer F.Cu) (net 18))
 (segment (start 138.05926 109.95142) (end 138.05926 112.30854) (width 1) (layer F.Cu) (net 18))
 (segment (start 140.60424 82.89144) (end 138.06424 85.43144) (width 1) (layer F.Cu) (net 18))
 (segment (start 140.60424 81.87944) (end 140.60424 82.89144) (width 1) (layer F.Cu) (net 18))
 (segment (start 138.06424 99.65944) (end 138.06424 85.43144) (width 1) (layer F.Cu) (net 18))
 (segment (start 165.4302 105.42524) (end 165.8302 105.42524) (width 0.25) (layer F.Cu) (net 5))
 (segment (start 161.43742 108.92038) (end 161.43742 105.19664) (width 1) (layer F.Cu) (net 5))
 (segment (start 161.43742 110.27664) (end 161.43742 109.10306) (width 1) (layer F.Cu) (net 5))
 (segment (start 161.43742 109.10306) (end 161.43742 108.92038) (width 0.25) (layer F.Cu) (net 5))
 (segment (start 165.0302 105.42524) (end 165.4302 105.42524) (width 0.25) (layer F.Cu) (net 5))
 (segment (start 161.66602 105.42524) (end 161.43742 105.19664) (width 0.25) (layer F.Cu) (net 5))
 (segment (start 165.4302 105.42524) (end 161.66602 105.42524) (width 1) (layer F.Cu) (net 5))
 (segment (start 162.01924 125.64644) (end 162.06724 125.69444) (width 0.25) (layer F.Cu) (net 9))
 (segment (start 161.96924 125.59644) (end 162.06724 125.69444) (width 0.25) (layer F.Cu) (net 9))
 (segment (start 162.06724 125.33894) (end 162.06724 125.69444) (width 0.25) (layer F.Cu) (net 9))
 (segment (start 162.06724 125.54204) (end 162.06724 125.69444) (width 0.25) (layer F.Cu) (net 9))
 (segment (start 162.06724 124.42844) (end 162.06724 125.69444) (width 1) (layer F.Cu) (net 9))
 (segment (start 162.06724 114.65454) (end 162.06724 124.42844) (width 1) (layer F.Cu) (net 9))
 (segment (start 165.87724 110.83544) (end 162.03264 114.68004) (width 1) (layer F.Cu) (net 9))
 (segment (start 166.48684 110.80994) (end 165.91184 110.80994) (width 1) (layer F.Cu) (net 9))
 (segment (start 164.33704 96.63694) (end 161.33064 99.64334) (width 1) (layer F.Cu) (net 9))
 (segment (start 164.91204 96.63694) (end 164.33704 96.63694) (width 1) (layer F.Cu) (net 9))
 (segment (start 161.33064 100.776684) (end 161.330818 100.776862) (width 0.25) (layer F.Cu) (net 9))
 (segment (start 166.81704 104.15524) (end 162.75304 104.15524) (width 0.5) (layer F.Cu) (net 9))
 (segment (start 168.597014 105.909814) (end 166.86784 104.18064) (width 0.5) (layer F.Cu) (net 9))
 (segment (start 157.21584 92.74844) (end 157.21584 98.71964) (width 1) (layer F.Cu) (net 9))
 (segment (start 162.54764 87.41664) (end 157.21584 92.74844) (width 1) (layer F.Cu) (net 9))
 (segment (start 163.99764 87.41664) (end 162.54764 87.41664) (width 1) (layer F.Cu) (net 9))
 (segment (start 161.35604 99.64842) (end 161.35604 102.83952) (width 1) (layer F.Cu) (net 9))
 (segment (start 168.597014 105.909814) (end 168.597014 108.699766) (width 0.5) (layer F.Cu) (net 9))
 (segment (start 168.54424 108.80344) (end 166.61389 110.73379) (width 0.5) (layer F.Cu) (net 9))
 (segment (start 161.33064 102.83444) (end 159.6644 101.1682) (width 1) (layer F.Cu) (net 9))
 (segment (start 157.21584 98.71964) (end 159.6644 101.1682) (width 1) (layer F.Cu) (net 9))
 (segment (start 159.6644 101.1682) (end 160.20034 101.70414) (width 1) (layer F.Cu) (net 9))
 (segment (start 161.43224 102.83444) (end 162.75304 104.15524) (width 0.5) (layer F.Cu) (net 9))
 (segment (start 161.33064 102.83444) (end 161.43224 102.83444) (width 0.25) (layer F.Cu) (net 9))
 (segment (start 165.0302 102.88524) (end 165.4302 102.88524) (width 0.25) (layer F.Cu) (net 3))
 (segment (start 166.8802 102.88524) (end 165.4302 102.88524) (width 0.5) (layer F.Cu) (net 3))
 (segment (start 169.76344 111.11474) (end 169.76344 110.57724) (width 0.25) (layer F.Cu) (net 3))
 (segment (start 169.76344 105.80624) (end 169.76344 111.11474) (width 0.5) (layer F.Cu) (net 3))
 (segment (start 165.8302 102.88524) (end 165.4302 102.88524) (width 0.25) (layer F.Cu) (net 3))
 (segment (start 170.83024 97.8852) (end 165.8302 102.88524) (width 1) (layer F.Cu) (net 3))
 (segment (start 170.83024 96.63694) (end 170.83024 97.8852) (width 1) (layer F.Cu) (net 3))
 (segment (start 169.76344 105.80624) (end 169.76344 104.43464) (width 0.5) (layer F.Cu) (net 3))
 (segment (start 168.21404 102.88524) (end 166.8802 102.88524) (width 0.5) (layer F.Cu) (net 3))
 (segment (start 169.76344 104.43464) (end 168.21404 102.88524) (width 0.5) (layer F.Cu) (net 3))
 (segment (start 173.4502 105.42524) (end 173.0502 105.42524) (width 0.25) (layer F.Cu) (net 4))
 (segment (start 173.101 105.47604) (end 173.0502 105.42524) (width 0.25) (layer F.Cu) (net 4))
 (segment (start 166.79164 112.68974) (end 166.48684 112.38494) (width 0.25) (layer F.Cu) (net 4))
 (segment (start 167.06184 112.38494) (end 169.76344 112.38494) (width 0.5) (layer F.Cu) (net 4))
 (segment (start 166.48684 112.38494) (end 167.06184 112.38494) (width 0.25) (layer F.Cu) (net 4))
 (segment (start 170.33844 112.38494) (end 169.76344 112.38494) (width 0.25) (layer F.Cu) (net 4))
 (segment (start 172.98924 112.38494) (end 170.33844 112.38494) (width 0.5) (layer F.Cu) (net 4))
 (segment (start 172.6502 105.42524) (end 171.26204 106.8134) (width 0.5) (layer F.Cu) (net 4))
 (segment (start 173.0502 105.42524) (end 172.6502 105.42524) (width 0.25) (layer F.Cu) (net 4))
 (segment (start 171.26204 110.65774) (end 172.98924 112.38494) (width 0.5) (layer F.Cu) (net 4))
 (segment (start 171.26204 106.8134) (end 171.26204 110.65774) (width 0.5) (layer F.Cu) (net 4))
 (segment (start 159.86242 110.27664) (end 152.56764 110.27664) (width 1) (layer F.Cu) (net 69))
 (segment (start 149.067688 110.27664) (end 150.33244 110.27664) (width 1) (layer F.Cu) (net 69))
 (segment (start 152.56764 110.27664) (end 150.33244 110.27664) (width 1) (layer F.Cu) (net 69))
 (segment (start 147.73656 110.75924) (end 148.585088 110.75924) (width 1) (layer F.Cu) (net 69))
 (segment (start 148.902504 110.441824) (end 148.585088 110.75924) (width 0.25) (layer F.Cu) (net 69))
 (segment (start 148.902504 110.441824) (end 149.067688 110.27664) (width 1) (layer F.Cu) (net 69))
 (segment (start 167.90924 95.06194) (end 170.83024 95.06194) (width 1) (layer F.Cu) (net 70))
 (segment (start 135.52424 101.23434) (end 136.48426 102.19436) (width 1) (layer F.Cu) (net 31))
 (segment (start 135.52424 99.65944) (end 135.52424 101.23434) (width 1) (layer F.Cu) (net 31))
 (segment (start 135.52424 86.7156) (end 135.52424 99.65944) (width 0.5) (layer F.Cu) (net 31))
 (segment (start 132.9436 84.13496) (end 135.52424 86.7156) (width 0.5) (layer F.Cu) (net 31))
 (segment (start 128.44272 84.13496) (end 132.9436 84.13496) (width 0.5) (layer F.Cu) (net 31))
 (segment (start 142.76324 78.70044) (end 141.63656 79.82712) (width 0.5) (layer F.Cu) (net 31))
 (segment (start 142.76324 77.43444) (end 142.76324 78.70044) (width 0.5) (layer F.Cu) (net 31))
 (segment (start 141.63656 79.82712) (end 129.33172 79.82712) (width 0.5) (layer F.Cu) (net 31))
 (segment (start 129.33172 79.82712) (end 127.52832 81.63052) (width 0.5) (layer F.Cu) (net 31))
 (segment (start 127.52832 81.63052) (end 127.52832 83.22056) (width 0.5) (layer F.Cu) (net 31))
 (segment (start 127.52832 83.22056) (end 128.44272 84.13496) (width 0.5) (layer F.Cu) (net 31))
 (segment (start 146.95424 80.48044) (end 146.95424 81.49244) (width 0.5) (layer F.Cu) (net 15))
 (segment (start 145.30324 78.70044) (end 146.95424 80.35144) (width 0.5) (layer F.Cu) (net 15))
 (segment (start 145.30324 77.43444) (end 145.30324 78.70044) (width 0.5) (layer F.Cu) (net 15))
 (segment (start 147.84324 77.43444) (end 147.84324 79.22768) (width 0.5) (layer F.Cu) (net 14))
 (segment (start 148.22424 79.60868) (end 148.22424 81.87944) (width 0.5) (layer F.Cu) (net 14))
 (segment (start 147.84324 79.22768) (end 148.22424 79.60868) (width 0.5) (layer F.Cu) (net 14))
 (segment (start 128.16224 89.49944) (end 121.50344 96.15824) (width 0.5) (layer F.Cu) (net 26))
 (segment (start 129.17424 89.49944) (end 128.16224 89.49944) (width 0.5) (layer F.Cu) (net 26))
 (segment (start 121.50344 99.79152) (end 119.40032 101.89464) (width 0.5) (layer F.Cu) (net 26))
 (segment (start 121.50344 96.15824) (end 121.50344 99.79152) (width 0.5) (layer F.Cu) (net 26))
 (segment (start 114.06124 101.89464) (end 119.40032 101.89464) (width 0.5) (layer F.Cu) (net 26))
 (segment (start 161.07674 84.87664) (end 161.07674 82.59064) (width 1) (layer F.Cu) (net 45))
 (segment (start 161.07674 84.87664) (end 163.99764 84.87664) (width 1) (layer F.Cu) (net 45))
 (segment (start 159.52724 82.56514) (end 159.50174 82.59064) (width 0.25) (layer F.Cu) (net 48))
 (segment (start 159.52724 77.43444) (end 159.52724 82.56514) (width 1) (layer F.Cu) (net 48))
 (segment (start 169.68724 78.70044) (end 167.97528 80.4124) (width 1) (layer F.Cu) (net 44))
 (segment (start 169.68724 77.43444) (end 169.68724 78.70044) (width 1) (layer F.Cu) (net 44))
 (segment (start 171.21764 87.41664) (end 171.61764 87.41664) (width 0.25) (layer F.Cu) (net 44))
 (segment (start 167.97528 80.4124) (end 167.97528 84.17428) (width 1) (layer F.Cu) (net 44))
 (segment (start 167.97528 85.49132) (end 167.97528 84.17428) (width 1) (layer F.Cu) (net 44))
 (segment (start 169.66184 87.26424) (end 169.15384 86.75624) (width 1) (layer F.Cu) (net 44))
 (segment (start 169.40784 86.95944) (end 167.95496 85.50656) (width 1) (layer F.Cu) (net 44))
 (segment (start 169.81424 87.41664) (end 169.66184 87.26424) (width 1) (layer F.Cu) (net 44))
 (segment (start 171.61764 87.41664) (end 169.81424 87.41664) (width 1) (layer F.Cu) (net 44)))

